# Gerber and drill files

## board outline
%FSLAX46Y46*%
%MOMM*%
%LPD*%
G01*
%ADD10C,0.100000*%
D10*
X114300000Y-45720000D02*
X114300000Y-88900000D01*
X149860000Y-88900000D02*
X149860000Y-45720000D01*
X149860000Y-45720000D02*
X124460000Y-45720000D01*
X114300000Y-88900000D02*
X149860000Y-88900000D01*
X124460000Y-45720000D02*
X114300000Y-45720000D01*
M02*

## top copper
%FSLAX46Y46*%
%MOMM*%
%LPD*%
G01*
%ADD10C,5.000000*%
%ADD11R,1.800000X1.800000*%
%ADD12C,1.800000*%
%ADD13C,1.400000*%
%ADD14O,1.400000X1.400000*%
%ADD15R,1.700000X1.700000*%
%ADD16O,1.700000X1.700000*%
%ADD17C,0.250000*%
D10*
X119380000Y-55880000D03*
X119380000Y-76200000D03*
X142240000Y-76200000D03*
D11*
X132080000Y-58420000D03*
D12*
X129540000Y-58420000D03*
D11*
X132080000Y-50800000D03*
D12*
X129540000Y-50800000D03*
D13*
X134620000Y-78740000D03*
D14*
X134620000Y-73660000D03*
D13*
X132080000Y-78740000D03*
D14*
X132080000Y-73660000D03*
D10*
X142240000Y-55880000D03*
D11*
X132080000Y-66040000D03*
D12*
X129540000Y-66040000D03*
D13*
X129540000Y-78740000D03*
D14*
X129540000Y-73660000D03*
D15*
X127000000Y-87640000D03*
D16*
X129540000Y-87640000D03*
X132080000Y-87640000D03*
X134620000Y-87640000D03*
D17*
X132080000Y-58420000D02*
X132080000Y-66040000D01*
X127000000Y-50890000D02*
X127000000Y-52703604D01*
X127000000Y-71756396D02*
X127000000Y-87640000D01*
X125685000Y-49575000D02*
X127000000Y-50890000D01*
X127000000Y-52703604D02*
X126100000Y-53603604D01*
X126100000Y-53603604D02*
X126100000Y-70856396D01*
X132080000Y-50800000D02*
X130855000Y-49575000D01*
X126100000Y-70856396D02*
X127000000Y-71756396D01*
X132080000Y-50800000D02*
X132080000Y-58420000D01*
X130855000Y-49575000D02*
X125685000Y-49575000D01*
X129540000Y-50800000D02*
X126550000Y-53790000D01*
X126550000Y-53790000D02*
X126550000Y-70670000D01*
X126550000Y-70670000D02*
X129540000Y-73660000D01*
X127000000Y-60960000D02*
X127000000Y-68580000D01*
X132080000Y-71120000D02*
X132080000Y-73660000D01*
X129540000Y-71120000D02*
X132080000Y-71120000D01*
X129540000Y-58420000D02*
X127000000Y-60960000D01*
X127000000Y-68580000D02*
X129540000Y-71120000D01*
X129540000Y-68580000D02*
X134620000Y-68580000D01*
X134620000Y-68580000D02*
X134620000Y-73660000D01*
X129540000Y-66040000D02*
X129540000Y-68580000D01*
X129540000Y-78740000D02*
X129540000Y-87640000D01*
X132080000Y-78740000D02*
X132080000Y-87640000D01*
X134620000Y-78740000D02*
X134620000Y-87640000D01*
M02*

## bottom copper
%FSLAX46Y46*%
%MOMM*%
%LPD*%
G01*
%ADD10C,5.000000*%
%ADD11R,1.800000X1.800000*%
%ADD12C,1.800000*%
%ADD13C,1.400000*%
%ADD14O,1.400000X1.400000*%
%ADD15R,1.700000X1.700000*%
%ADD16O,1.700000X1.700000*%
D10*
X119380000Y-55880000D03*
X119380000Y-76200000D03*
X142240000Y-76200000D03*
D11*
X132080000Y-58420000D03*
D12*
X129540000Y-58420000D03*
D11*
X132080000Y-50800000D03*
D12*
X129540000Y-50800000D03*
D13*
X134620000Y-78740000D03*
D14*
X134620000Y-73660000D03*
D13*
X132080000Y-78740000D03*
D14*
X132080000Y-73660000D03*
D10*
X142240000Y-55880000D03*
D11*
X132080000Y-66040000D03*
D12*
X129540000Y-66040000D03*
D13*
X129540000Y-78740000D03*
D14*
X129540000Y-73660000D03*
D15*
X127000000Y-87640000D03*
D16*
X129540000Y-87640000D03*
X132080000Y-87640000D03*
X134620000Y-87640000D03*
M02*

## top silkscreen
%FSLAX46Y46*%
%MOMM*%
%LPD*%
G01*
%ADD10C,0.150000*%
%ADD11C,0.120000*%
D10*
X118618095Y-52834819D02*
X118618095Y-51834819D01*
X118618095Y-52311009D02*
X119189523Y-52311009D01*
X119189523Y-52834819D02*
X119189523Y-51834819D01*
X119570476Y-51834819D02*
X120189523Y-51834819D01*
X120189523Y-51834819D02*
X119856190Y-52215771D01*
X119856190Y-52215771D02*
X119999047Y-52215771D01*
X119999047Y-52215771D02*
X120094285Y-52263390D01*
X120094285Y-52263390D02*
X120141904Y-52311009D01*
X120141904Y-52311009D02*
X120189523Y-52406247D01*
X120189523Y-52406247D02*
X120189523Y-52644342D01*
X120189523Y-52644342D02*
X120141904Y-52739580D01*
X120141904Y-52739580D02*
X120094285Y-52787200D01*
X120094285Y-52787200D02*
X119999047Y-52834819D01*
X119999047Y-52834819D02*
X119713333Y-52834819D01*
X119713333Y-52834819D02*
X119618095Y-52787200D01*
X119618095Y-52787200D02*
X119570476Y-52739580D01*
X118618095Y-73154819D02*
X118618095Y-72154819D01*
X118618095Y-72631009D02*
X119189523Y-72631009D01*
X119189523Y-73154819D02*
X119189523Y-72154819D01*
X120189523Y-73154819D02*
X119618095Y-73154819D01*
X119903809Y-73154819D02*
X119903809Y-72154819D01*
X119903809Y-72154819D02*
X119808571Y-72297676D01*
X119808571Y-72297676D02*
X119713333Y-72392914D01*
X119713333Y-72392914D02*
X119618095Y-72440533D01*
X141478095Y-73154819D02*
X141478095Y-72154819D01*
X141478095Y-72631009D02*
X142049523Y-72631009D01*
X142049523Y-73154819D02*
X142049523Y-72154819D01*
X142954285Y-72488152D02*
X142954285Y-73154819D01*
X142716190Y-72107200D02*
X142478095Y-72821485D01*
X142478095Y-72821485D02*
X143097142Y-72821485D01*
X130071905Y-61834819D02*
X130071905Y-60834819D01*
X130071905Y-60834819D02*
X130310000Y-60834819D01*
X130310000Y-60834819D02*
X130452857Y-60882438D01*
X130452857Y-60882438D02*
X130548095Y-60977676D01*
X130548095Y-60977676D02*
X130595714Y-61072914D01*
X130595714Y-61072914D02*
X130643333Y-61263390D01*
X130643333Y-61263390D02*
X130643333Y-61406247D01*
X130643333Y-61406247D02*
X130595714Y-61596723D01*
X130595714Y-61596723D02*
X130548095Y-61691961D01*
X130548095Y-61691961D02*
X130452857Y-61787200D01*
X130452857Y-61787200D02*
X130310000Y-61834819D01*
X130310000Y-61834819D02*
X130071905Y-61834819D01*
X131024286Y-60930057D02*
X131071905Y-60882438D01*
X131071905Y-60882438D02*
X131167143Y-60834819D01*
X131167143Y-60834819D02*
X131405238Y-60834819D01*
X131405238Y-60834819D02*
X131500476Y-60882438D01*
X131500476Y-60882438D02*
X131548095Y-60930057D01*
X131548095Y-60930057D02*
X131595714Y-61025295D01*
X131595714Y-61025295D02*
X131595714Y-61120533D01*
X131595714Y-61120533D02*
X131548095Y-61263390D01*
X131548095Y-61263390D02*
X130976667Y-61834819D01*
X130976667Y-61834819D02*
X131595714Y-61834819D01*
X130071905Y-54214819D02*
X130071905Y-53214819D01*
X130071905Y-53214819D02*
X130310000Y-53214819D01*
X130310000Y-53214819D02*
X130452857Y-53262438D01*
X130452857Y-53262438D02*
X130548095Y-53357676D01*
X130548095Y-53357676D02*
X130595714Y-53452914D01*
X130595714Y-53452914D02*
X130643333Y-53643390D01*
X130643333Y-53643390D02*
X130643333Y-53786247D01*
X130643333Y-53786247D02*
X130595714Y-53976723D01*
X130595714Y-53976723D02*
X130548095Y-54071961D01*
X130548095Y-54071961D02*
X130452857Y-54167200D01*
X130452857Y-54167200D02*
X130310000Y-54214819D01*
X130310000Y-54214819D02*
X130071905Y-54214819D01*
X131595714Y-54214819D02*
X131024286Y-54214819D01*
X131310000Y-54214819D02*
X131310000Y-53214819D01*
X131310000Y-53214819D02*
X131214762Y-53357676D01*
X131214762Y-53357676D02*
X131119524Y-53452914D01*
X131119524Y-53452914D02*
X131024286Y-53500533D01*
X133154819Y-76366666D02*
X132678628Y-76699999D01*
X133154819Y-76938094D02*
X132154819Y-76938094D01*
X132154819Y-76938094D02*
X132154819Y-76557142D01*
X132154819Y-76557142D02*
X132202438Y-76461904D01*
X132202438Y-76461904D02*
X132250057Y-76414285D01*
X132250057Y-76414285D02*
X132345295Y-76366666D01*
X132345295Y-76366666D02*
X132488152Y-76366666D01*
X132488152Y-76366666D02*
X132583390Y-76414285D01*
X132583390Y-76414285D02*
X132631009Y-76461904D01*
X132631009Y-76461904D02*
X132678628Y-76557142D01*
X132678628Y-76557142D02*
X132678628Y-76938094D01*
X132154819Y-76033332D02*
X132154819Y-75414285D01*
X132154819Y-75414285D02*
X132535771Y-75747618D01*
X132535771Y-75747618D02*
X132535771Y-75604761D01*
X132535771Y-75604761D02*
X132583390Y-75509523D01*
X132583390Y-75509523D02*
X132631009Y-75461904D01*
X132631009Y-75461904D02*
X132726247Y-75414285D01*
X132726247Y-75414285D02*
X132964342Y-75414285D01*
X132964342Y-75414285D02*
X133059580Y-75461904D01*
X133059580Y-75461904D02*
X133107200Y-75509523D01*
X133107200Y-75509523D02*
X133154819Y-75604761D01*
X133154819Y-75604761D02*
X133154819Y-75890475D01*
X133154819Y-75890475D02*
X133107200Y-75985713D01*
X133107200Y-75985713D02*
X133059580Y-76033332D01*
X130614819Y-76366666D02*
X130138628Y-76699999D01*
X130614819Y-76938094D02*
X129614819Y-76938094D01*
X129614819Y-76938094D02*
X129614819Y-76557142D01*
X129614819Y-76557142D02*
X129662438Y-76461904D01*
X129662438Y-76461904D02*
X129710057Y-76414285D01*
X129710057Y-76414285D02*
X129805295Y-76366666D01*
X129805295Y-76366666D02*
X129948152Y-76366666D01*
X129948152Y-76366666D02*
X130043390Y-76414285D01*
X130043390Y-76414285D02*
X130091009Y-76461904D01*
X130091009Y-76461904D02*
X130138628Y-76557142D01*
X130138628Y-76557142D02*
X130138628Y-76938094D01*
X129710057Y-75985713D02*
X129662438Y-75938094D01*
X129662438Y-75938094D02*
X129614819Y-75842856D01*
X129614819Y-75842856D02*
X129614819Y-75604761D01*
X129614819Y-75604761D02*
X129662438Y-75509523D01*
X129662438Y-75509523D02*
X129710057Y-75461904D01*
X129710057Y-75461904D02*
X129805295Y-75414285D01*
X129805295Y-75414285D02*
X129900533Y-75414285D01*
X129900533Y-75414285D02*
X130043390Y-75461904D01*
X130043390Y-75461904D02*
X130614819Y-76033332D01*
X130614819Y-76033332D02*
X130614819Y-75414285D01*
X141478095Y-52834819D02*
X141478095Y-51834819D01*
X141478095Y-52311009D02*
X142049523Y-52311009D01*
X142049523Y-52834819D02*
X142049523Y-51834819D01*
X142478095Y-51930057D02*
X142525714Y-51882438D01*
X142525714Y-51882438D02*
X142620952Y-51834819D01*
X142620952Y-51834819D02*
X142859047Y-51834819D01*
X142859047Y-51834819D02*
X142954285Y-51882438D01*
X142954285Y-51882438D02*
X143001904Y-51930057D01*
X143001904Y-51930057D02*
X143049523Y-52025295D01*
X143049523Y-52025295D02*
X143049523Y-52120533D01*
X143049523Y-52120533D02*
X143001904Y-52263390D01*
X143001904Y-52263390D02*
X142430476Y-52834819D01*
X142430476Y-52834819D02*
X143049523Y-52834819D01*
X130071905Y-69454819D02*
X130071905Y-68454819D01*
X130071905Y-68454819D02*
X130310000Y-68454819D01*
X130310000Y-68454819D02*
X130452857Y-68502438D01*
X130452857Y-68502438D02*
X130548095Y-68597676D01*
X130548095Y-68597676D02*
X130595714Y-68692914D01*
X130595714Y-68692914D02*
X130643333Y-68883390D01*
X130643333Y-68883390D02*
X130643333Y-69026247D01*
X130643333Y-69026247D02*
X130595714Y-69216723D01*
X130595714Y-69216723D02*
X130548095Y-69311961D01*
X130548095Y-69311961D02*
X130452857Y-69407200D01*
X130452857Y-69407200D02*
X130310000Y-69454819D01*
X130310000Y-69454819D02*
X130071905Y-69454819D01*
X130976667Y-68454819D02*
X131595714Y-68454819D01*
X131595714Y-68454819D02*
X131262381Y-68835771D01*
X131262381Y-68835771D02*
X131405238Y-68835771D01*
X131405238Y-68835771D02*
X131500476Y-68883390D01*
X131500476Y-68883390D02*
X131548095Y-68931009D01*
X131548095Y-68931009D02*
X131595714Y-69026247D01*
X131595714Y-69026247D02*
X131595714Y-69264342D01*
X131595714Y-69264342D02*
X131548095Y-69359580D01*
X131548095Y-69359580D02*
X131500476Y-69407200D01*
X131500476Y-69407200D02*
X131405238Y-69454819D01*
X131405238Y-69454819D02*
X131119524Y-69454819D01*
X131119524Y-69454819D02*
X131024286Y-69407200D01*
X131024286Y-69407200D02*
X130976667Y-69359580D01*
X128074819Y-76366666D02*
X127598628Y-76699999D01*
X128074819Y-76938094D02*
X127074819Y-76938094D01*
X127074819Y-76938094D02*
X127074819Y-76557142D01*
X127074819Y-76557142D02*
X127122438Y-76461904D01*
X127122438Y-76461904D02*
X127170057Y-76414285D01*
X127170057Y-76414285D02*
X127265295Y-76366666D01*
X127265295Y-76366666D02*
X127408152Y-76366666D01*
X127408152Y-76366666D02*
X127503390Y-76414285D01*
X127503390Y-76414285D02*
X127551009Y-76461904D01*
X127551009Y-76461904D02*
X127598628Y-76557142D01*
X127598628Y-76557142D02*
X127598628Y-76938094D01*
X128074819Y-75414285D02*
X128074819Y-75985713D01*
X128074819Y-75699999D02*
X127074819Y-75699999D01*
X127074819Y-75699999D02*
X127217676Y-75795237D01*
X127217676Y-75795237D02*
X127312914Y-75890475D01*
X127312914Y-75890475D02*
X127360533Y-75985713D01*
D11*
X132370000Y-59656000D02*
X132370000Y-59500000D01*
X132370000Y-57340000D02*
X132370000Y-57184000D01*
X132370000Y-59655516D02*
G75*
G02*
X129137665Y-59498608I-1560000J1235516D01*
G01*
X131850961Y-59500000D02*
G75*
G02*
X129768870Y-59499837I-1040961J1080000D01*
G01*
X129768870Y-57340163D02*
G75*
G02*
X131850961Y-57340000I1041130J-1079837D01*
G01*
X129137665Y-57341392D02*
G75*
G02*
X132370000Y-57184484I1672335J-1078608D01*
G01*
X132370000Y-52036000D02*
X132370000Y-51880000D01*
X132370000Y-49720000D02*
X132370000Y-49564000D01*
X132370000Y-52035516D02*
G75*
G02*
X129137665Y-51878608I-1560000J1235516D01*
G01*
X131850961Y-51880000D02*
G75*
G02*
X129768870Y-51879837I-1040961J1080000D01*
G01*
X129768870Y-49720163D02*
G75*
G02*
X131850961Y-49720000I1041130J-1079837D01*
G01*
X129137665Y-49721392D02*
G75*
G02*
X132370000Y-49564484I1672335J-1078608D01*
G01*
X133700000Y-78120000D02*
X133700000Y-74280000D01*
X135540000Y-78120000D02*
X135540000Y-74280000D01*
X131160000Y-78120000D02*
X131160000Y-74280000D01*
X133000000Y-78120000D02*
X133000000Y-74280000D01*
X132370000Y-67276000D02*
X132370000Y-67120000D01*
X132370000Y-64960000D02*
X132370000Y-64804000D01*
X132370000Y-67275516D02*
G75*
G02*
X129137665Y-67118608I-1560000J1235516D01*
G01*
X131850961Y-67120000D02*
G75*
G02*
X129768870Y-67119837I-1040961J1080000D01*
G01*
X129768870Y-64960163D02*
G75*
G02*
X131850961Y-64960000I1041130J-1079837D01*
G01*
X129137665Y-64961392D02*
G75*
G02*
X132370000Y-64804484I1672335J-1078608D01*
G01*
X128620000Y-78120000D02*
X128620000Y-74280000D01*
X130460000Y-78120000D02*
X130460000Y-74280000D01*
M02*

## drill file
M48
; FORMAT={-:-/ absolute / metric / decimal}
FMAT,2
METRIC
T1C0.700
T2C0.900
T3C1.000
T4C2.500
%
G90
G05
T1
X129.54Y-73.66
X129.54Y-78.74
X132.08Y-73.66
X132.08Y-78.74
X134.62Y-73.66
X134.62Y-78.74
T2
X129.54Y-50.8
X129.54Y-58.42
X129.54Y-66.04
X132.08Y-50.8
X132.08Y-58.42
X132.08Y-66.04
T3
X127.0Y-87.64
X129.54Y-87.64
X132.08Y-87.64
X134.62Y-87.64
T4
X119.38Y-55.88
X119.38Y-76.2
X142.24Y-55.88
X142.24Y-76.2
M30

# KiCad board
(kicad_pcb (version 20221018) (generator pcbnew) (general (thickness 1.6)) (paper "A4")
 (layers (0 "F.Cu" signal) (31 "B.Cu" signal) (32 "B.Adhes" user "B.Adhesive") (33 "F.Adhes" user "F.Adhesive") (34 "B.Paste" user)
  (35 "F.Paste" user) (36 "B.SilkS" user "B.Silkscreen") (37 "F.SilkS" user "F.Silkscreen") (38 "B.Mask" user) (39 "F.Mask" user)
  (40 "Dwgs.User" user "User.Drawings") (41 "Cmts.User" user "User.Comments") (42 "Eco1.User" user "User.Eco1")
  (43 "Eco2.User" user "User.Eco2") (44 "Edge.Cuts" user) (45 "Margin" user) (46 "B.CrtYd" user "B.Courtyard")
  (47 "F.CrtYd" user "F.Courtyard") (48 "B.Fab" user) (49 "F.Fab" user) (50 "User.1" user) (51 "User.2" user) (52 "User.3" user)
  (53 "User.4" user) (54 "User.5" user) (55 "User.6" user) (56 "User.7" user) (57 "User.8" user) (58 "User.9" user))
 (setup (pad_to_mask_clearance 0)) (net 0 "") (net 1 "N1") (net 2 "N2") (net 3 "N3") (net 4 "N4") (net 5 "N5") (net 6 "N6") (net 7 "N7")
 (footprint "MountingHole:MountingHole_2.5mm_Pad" (layer "F.Cu") (at 119.38 55.88)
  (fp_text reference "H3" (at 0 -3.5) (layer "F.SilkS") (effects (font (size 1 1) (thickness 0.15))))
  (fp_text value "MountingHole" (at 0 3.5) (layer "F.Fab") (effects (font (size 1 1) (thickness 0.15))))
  (pad "1" thru_hole circle (at 0 0) (size 5 5) (drill 2.5) (layers "*.Cu" "*.Mask")))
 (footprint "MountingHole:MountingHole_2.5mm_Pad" (layer "F.Cu") (at 119.38 76.2)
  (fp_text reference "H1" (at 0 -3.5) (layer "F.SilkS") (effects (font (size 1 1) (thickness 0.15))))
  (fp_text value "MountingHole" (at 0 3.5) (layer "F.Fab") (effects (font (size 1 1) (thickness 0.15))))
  (pad "1" thru_hole circle (at 0 0) (size 5 5) (drill 2.5) (layers "*.Cu" "*.Mask")))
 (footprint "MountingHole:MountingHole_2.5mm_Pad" (layer "F.Cu") (at 142.24 76.2)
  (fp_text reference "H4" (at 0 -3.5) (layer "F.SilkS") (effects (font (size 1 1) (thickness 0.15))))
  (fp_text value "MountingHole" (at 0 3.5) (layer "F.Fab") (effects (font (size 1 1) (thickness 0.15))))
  (pad "1" thru_hole circle (at 0 0) (size 5 5) (drill 2.5) (layers "*.Cu" "*.Mask")))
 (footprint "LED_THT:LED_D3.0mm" (layer "F.Cu") (at 132.08 58.42 180)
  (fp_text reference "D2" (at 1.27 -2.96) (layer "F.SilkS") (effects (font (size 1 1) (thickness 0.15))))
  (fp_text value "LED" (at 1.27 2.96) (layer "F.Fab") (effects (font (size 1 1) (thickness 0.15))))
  (fp_line (start -0.29 -1.236) (end -0.29 -1.08) (stroke (width 0.12) (type solid)) (layer "F.SilkS"))
  (fp_line (start -0.29 1.08) (end -0.29 1.236) (stroke (width 0.12) (type solid)) (layer "F.SilkS"))
  (fp_arc (start -0.29 -1.235516) (mid 1.366487 -1.987659) (end 2.942335 -1.078608) (stroke (width 0.12) (type solid)) (layer "F.SilkS"))
  (fp_arc (start 0.229039 -1.08) (mid 1.270117 -1.5) (end 2.31113 -1.079837) (stroke (width 0.12) (type solid)) (layer "F.SilkS"))
  (fp_arc (start 2.31113 1.079837) (mid 1.270117 1.5) (end 0.229039 1.08) (stroke (width 0.12) (type solid)) (layer "F.SilkS"))
  (fp_arc (start 2.942335 1.078608) (mid 1.366487 1.987659) (end -0.29 1.235516) (stroke (width 0.12) (type solid)) (layer "F.SilkS"))
  (pad "1" thru_hole rect (at 0 0 180) (size 1.8 1.8) (drill 0.9) (layers "*.Cu" "*.Mask") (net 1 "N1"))
  (pad "2" thru_hole circle (at 2.54 0 180) (size 1.8 1.8) (drill 0.9) (layers "*.Cu" "*.Mask") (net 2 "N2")))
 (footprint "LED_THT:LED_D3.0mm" (layer "F.Cu") (at 132.08 50.8 180)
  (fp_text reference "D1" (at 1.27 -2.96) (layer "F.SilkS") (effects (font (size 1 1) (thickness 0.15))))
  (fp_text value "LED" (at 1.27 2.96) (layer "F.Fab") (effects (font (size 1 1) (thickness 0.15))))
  (fp_line (start -0.29 -1.236) (end -0.29 -1.08) (stroke (width 0.12) (type solid)) (layer "F.SilkS"))
  (fp_line (start -0.29 1.08) (end -0.29 1.236) (stroke (width 0.12) (type solid)) (layer "F.SilkS"))
  (fp_arc (start -0.29 -1.235516) (mid 1.366487 -1.987659) (end 2.942335 -1.078608) (stroke (width 0.12) (type solid)) (layer "F.SilkS"))
  (fp_arc (start 0.229039 -1.08) (mid 1.270117 -1.5) (end 2.31113 -1.079837) (stroke (width 0.12) (type solid)) (layer "F.SilkS"))
  (fp_arc (start 2.31113 1.079837) (mid 1.270117 1.5) (end 0.229039 1.08) (stroke (width 0.12) (type solid)) (layer "F.SilkS"))
  (fp_arc (start 2.942335 1.078608) (mid 1.366487 1.987659) (end -0.29 1.235516) (stroke (width 0.12) (type solid)) (layer "F.SilkS"))
  (pad "1" thru_hole rect (at 0 0 180) (size 1.8 1.8) (drill 0.9) (layers "*.Cu" "*.Mask") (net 1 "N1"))
  (pad "2" thru_hole circle (at 2.54 0 180) (size 1.8 1.8) (drill 0.9) (layers "*.Cu" "*.Mask") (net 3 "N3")))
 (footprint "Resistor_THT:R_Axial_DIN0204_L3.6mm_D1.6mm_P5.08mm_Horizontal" (layer "F.Cu") (at 134.62 78.74 90)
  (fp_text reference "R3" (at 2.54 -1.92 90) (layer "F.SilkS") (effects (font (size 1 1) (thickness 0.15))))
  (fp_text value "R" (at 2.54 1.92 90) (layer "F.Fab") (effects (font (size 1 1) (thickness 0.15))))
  (fp_line (start 0.62 -0.92) (end 4.46 -0.92) (stroke (width 0.12) (type solid)) (layer "F.SilkS"))
  (fp_line (start 0.62 0.92) (end 4.46 0.92) (stroke (width 0.12) (type solid)) (layer "F.SilkS"))
  (pad "1" thru_hole circle (at 0 0 90) (size 1.4 1.4) (drill 0.7) (layers "*.Cu" "*.Mask") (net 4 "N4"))
  (pad "2" thru_hole oval (at 5.08 0 90) (size 1.4 1.4) (drill 0.7) (layers "*.Cu" "*.Mask") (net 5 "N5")))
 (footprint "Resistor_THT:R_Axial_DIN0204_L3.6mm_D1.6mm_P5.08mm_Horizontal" (layer "F.Cu") (at 132.08 78.74 90)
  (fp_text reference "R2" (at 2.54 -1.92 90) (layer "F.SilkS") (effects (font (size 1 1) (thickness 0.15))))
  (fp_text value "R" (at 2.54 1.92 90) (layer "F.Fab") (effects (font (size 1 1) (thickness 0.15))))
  (fp_line (start 0.62 -0.92) (end 4.46 -0.92) (stroke (width 0.12) (type solid)) (layer "F.SilkS"))
  (fp_line (start 0.62 0.92) (end 4.46 0.92) (stroke (width 0.12) (type solid)) (layer "F.SilkS"))
  (pad "1" thru_hole circle (at 0 0 90) (size 1.4 1.4) (drill 0.7) (layers "*.Cu" "*.Mask") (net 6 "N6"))
  (pad "2" thru_hole oval (at 5.08 0 90) (size 1.4 1.4) (drill 0.7) (layers "*.Cu" "*.Mask") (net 2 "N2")))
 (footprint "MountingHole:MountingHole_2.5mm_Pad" (layer "F.Cu") (at 142.24 55.88)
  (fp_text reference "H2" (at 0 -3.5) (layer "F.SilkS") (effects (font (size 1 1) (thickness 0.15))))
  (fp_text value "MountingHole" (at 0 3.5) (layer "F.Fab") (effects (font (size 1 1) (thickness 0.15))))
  (pad "1" thru_hole circle (at 0 0) (size 5 5) (drill 2.5) (layers "*.Cu" "*.Mask")))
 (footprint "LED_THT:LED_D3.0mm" (layer "F.Cu") (at 132.08 66.04 180)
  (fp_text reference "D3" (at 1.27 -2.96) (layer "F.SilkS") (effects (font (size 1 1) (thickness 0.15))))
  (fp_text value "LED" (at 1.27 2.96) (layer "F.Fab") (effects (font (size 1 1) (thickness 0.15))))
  (fp_line (start -0.29 -1.236) (end -0.29 -1.08) (stroke (width 0.12) (type solid)) (layer "F.SilkS"))
  (fp_line (start -0.29 1.08) (end -0.29 1.236) (stroke (width 0.12) (type solid)) (layer "F.SilkS"))
  (fp_arc (start -0.29 -1.235516) (mid 1.366487 -1.987659) (end 2.942335 -1.078608) (stroke (width 0.12) (type solid)) (layer "F.SilkS"))
  (fp_arc (start 0.229039 -1.08) (mid 1.270117 -1.5) (end 2.31113 -1.079837) (stroke (width 0.12) (type solid)) (layer "F.SilkS"))
  (fp_arc (start 2.31113 1.079837) (mid 1.270117 1.5) (end 0.229039 1.08) (stroke (width 0.12) (type solid)) (layer "F.SilkS"))
  (fp_arc (start 2.942335 1.078608) (mid 1.366487 1.987659) (end -0.29 1.235516) (stroke (width 0.12) (type solid)) (layer "F.SilkS"))
  (pad "1" thru_hole rect (at 0 0 180) (size 1.8 1.8) (drill 0.9) (layers "*.Cu" "*.Mask") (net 1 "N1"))
  (pad "2" thru_hole circle (at 2.54 0 180) (size 1.8 1.8) (drill 0.9) (layers "*.Cu" "*.Mask") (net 5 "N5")))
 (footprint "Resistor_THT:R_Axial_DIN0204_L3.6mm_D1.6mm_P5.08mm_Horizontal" (layer "F.Cu") (at 129.54 78.74 90)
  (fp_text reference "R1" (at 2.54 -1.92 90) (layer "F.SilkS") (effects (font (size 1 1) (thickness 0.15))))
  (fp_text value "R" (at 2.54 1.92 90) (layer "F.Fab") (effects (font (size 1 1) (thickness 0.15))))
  (fp_line (start 0.62 -0.92) (end 4.46 -0.92) (stroke (width 0.12) (type solid)) (layer "F.SilkS"))
  (fp_line (start 0.62 0.92) (end 4.46 0.92) (stroke (width 0.12) (type solid)) (layer "F.SilkS"))
  (pad "1" thru_hole circle (at 0 0 90) (size 1.4 1.4) (drill 0.7) (layers "*.Cu" "*.Mask") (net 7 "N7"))
  (pad "2" thru_hole oval (at 5.08 0 90) (size 1.4 1.4) (drill 0.7) (layers "*.Cu" "*.Mask") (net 3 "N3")))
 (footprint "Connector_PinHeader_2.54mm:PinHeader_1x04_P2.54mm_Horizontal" (layer "B.Cu") (at 127 87.64 -90)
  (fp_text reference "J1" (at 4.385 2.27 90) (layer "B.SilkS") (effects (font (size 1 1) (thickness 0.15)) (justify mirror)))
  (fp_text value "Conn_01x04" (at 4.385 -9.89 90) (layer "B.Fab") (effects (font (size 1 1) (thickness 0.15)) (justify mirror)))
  (pad "1" thru_hole rect (at 0 0 270) (size 1.7 1.7) (drill 1) (layers "*.Cu" "*.Mask") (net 1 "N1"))
  (pad "2" thru_hole oval (at 0 -2.54 270) (size 1.7 1.7) (drill 1) (layers "*.Cu" "*.Mask") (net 7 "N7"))
  (pad "3" thru_hole oval (at 0 -5.08 270) (size 1.7 1.7) (drill 1) (layers "*.Cu" "*.Mask") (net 6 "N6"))
  (pad "4" thru_hole oval (at 0 -7.62 270) (size 1.7 1.7) (drill 1) (layers "*.Cu" "*.Mask") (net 4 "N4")))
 (gr_line (start 114.3 45.72) (end 114.3 88.9) (stroke (width 0.1) (type default)) (layer "Edge.Cuts"))
 (gr_line (start 149.86 88.9) (end 149.86 45.72) (stroke (width 0.1) (type default)) (layer "Edge.Cuts"))
 (gr_line (start 149.86 45.72) (end 124.46 45.72) (stroke (width 0.1) (type default)) (layer "Edge.Cuts"))
 (gr_line (start 114.3 88.9) (end 149.86 88.9) (stroke (width 0.1) (type default)) (layer "Edge.Cuts"))
 (gr_line (start 124.46 45.72) (end 114.3 45.72) (stroke (width 0.1) (type default)) (layer "Edge.Cuts"))
 (segment (start 132.08 58.42) (end 132.08 66.04) (width 0.25) (layer "F.Cu") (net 1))
 (segment (start 127 50.89) (end 127 52.703604) (width 0.25) (layer "F.Cu") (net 1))
 (segment (start 127 71.756396) (end 127 87.64) (width 0.25) (layer "F.Cu") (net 1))
 (segment (start 125.685 49.575) (end 127 50.89) (width 0.25) (layer "F.Cu") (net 1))
 (segment (start 127 52.703604) (end 126.1 53.603604) (width 0.25) (layer "F.Cu") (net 1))
 (segment (start 126.1 53.603604) (end 126.1 70.856396) (width 0.25) (layer "F.Cu") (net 1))
 (segment (start 132.08 50.8) (end 130.855 49.575) (width 0.25) (layer "F.Cu") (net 1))
 (segment (start 126.1 70.856396) (end 127 71.756396) (width 0.25) (layer "F.Cu") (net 1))
 (segment (start 132.08 50.8) (end 132.08 58.42) (width 0.25) (layer "F.Cu") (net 1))
 (segment (start 130.855 49.575) (end 125.685 49.575) (width 0.25) (layer "F.Cu") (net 1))
 (segment (start 129.54 50.8) (end 126.55 53.79) (width 0.25) (layer "F.Cu") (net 3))
 (segment (start 126.55 53.79) (end 126.55 70.67) (width 0.25) (layer "F.Cu") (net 3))
 (segment (start 126.55 70.67) (end 129.54 73.66) (width 0.25) (layer "F.Cu") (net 3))
 (segment (start 127 60.96) (end 127 68.58) (width 0.25) (layer "F.Cu") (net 2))
 (segment (start 132.08 71.12) (end 132.08 73.66) (width 0.25) (layer "F.Cu") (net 2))
 (segment (start 129.54 71.12) (end 132.08 71.12) (width 0.25) (layer "F.Cu") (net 2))
 (segment (start 129.54 58.42) (end 127 60.96) (width 0.25) (layer "F.Cu") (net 2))
 (segment (start 127 68.58) (end 129.54 71.12) (width 0.25) (layer "F.Cu") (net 2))
 (segment (start 129.54 68.58) (end 134.62 68.58) (width 0.25) (layer "F.Cu") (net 5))
 (segment (start 134.62 68.58) (end 134.62 73.66) (width 0.25) (layer "F.Cu") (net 5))
 (segment (start 129.54 66.04) (end 129.54 68.58) (width 0.25) (layer "F.Cu") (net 5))
 (segment (start 129.54 78.74) (end 129.54 87.64) (width 0.25) (layer "F.Cu") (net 7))
 (segment (start 132.08 78.74) (end 132.08 87.64) (width 0.25) (layer "F.Cu") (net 6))
 (segment (start 134.62 78.74) (end 134.62 87.64) (width 0.25) (layer "F.Cu") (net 4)))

